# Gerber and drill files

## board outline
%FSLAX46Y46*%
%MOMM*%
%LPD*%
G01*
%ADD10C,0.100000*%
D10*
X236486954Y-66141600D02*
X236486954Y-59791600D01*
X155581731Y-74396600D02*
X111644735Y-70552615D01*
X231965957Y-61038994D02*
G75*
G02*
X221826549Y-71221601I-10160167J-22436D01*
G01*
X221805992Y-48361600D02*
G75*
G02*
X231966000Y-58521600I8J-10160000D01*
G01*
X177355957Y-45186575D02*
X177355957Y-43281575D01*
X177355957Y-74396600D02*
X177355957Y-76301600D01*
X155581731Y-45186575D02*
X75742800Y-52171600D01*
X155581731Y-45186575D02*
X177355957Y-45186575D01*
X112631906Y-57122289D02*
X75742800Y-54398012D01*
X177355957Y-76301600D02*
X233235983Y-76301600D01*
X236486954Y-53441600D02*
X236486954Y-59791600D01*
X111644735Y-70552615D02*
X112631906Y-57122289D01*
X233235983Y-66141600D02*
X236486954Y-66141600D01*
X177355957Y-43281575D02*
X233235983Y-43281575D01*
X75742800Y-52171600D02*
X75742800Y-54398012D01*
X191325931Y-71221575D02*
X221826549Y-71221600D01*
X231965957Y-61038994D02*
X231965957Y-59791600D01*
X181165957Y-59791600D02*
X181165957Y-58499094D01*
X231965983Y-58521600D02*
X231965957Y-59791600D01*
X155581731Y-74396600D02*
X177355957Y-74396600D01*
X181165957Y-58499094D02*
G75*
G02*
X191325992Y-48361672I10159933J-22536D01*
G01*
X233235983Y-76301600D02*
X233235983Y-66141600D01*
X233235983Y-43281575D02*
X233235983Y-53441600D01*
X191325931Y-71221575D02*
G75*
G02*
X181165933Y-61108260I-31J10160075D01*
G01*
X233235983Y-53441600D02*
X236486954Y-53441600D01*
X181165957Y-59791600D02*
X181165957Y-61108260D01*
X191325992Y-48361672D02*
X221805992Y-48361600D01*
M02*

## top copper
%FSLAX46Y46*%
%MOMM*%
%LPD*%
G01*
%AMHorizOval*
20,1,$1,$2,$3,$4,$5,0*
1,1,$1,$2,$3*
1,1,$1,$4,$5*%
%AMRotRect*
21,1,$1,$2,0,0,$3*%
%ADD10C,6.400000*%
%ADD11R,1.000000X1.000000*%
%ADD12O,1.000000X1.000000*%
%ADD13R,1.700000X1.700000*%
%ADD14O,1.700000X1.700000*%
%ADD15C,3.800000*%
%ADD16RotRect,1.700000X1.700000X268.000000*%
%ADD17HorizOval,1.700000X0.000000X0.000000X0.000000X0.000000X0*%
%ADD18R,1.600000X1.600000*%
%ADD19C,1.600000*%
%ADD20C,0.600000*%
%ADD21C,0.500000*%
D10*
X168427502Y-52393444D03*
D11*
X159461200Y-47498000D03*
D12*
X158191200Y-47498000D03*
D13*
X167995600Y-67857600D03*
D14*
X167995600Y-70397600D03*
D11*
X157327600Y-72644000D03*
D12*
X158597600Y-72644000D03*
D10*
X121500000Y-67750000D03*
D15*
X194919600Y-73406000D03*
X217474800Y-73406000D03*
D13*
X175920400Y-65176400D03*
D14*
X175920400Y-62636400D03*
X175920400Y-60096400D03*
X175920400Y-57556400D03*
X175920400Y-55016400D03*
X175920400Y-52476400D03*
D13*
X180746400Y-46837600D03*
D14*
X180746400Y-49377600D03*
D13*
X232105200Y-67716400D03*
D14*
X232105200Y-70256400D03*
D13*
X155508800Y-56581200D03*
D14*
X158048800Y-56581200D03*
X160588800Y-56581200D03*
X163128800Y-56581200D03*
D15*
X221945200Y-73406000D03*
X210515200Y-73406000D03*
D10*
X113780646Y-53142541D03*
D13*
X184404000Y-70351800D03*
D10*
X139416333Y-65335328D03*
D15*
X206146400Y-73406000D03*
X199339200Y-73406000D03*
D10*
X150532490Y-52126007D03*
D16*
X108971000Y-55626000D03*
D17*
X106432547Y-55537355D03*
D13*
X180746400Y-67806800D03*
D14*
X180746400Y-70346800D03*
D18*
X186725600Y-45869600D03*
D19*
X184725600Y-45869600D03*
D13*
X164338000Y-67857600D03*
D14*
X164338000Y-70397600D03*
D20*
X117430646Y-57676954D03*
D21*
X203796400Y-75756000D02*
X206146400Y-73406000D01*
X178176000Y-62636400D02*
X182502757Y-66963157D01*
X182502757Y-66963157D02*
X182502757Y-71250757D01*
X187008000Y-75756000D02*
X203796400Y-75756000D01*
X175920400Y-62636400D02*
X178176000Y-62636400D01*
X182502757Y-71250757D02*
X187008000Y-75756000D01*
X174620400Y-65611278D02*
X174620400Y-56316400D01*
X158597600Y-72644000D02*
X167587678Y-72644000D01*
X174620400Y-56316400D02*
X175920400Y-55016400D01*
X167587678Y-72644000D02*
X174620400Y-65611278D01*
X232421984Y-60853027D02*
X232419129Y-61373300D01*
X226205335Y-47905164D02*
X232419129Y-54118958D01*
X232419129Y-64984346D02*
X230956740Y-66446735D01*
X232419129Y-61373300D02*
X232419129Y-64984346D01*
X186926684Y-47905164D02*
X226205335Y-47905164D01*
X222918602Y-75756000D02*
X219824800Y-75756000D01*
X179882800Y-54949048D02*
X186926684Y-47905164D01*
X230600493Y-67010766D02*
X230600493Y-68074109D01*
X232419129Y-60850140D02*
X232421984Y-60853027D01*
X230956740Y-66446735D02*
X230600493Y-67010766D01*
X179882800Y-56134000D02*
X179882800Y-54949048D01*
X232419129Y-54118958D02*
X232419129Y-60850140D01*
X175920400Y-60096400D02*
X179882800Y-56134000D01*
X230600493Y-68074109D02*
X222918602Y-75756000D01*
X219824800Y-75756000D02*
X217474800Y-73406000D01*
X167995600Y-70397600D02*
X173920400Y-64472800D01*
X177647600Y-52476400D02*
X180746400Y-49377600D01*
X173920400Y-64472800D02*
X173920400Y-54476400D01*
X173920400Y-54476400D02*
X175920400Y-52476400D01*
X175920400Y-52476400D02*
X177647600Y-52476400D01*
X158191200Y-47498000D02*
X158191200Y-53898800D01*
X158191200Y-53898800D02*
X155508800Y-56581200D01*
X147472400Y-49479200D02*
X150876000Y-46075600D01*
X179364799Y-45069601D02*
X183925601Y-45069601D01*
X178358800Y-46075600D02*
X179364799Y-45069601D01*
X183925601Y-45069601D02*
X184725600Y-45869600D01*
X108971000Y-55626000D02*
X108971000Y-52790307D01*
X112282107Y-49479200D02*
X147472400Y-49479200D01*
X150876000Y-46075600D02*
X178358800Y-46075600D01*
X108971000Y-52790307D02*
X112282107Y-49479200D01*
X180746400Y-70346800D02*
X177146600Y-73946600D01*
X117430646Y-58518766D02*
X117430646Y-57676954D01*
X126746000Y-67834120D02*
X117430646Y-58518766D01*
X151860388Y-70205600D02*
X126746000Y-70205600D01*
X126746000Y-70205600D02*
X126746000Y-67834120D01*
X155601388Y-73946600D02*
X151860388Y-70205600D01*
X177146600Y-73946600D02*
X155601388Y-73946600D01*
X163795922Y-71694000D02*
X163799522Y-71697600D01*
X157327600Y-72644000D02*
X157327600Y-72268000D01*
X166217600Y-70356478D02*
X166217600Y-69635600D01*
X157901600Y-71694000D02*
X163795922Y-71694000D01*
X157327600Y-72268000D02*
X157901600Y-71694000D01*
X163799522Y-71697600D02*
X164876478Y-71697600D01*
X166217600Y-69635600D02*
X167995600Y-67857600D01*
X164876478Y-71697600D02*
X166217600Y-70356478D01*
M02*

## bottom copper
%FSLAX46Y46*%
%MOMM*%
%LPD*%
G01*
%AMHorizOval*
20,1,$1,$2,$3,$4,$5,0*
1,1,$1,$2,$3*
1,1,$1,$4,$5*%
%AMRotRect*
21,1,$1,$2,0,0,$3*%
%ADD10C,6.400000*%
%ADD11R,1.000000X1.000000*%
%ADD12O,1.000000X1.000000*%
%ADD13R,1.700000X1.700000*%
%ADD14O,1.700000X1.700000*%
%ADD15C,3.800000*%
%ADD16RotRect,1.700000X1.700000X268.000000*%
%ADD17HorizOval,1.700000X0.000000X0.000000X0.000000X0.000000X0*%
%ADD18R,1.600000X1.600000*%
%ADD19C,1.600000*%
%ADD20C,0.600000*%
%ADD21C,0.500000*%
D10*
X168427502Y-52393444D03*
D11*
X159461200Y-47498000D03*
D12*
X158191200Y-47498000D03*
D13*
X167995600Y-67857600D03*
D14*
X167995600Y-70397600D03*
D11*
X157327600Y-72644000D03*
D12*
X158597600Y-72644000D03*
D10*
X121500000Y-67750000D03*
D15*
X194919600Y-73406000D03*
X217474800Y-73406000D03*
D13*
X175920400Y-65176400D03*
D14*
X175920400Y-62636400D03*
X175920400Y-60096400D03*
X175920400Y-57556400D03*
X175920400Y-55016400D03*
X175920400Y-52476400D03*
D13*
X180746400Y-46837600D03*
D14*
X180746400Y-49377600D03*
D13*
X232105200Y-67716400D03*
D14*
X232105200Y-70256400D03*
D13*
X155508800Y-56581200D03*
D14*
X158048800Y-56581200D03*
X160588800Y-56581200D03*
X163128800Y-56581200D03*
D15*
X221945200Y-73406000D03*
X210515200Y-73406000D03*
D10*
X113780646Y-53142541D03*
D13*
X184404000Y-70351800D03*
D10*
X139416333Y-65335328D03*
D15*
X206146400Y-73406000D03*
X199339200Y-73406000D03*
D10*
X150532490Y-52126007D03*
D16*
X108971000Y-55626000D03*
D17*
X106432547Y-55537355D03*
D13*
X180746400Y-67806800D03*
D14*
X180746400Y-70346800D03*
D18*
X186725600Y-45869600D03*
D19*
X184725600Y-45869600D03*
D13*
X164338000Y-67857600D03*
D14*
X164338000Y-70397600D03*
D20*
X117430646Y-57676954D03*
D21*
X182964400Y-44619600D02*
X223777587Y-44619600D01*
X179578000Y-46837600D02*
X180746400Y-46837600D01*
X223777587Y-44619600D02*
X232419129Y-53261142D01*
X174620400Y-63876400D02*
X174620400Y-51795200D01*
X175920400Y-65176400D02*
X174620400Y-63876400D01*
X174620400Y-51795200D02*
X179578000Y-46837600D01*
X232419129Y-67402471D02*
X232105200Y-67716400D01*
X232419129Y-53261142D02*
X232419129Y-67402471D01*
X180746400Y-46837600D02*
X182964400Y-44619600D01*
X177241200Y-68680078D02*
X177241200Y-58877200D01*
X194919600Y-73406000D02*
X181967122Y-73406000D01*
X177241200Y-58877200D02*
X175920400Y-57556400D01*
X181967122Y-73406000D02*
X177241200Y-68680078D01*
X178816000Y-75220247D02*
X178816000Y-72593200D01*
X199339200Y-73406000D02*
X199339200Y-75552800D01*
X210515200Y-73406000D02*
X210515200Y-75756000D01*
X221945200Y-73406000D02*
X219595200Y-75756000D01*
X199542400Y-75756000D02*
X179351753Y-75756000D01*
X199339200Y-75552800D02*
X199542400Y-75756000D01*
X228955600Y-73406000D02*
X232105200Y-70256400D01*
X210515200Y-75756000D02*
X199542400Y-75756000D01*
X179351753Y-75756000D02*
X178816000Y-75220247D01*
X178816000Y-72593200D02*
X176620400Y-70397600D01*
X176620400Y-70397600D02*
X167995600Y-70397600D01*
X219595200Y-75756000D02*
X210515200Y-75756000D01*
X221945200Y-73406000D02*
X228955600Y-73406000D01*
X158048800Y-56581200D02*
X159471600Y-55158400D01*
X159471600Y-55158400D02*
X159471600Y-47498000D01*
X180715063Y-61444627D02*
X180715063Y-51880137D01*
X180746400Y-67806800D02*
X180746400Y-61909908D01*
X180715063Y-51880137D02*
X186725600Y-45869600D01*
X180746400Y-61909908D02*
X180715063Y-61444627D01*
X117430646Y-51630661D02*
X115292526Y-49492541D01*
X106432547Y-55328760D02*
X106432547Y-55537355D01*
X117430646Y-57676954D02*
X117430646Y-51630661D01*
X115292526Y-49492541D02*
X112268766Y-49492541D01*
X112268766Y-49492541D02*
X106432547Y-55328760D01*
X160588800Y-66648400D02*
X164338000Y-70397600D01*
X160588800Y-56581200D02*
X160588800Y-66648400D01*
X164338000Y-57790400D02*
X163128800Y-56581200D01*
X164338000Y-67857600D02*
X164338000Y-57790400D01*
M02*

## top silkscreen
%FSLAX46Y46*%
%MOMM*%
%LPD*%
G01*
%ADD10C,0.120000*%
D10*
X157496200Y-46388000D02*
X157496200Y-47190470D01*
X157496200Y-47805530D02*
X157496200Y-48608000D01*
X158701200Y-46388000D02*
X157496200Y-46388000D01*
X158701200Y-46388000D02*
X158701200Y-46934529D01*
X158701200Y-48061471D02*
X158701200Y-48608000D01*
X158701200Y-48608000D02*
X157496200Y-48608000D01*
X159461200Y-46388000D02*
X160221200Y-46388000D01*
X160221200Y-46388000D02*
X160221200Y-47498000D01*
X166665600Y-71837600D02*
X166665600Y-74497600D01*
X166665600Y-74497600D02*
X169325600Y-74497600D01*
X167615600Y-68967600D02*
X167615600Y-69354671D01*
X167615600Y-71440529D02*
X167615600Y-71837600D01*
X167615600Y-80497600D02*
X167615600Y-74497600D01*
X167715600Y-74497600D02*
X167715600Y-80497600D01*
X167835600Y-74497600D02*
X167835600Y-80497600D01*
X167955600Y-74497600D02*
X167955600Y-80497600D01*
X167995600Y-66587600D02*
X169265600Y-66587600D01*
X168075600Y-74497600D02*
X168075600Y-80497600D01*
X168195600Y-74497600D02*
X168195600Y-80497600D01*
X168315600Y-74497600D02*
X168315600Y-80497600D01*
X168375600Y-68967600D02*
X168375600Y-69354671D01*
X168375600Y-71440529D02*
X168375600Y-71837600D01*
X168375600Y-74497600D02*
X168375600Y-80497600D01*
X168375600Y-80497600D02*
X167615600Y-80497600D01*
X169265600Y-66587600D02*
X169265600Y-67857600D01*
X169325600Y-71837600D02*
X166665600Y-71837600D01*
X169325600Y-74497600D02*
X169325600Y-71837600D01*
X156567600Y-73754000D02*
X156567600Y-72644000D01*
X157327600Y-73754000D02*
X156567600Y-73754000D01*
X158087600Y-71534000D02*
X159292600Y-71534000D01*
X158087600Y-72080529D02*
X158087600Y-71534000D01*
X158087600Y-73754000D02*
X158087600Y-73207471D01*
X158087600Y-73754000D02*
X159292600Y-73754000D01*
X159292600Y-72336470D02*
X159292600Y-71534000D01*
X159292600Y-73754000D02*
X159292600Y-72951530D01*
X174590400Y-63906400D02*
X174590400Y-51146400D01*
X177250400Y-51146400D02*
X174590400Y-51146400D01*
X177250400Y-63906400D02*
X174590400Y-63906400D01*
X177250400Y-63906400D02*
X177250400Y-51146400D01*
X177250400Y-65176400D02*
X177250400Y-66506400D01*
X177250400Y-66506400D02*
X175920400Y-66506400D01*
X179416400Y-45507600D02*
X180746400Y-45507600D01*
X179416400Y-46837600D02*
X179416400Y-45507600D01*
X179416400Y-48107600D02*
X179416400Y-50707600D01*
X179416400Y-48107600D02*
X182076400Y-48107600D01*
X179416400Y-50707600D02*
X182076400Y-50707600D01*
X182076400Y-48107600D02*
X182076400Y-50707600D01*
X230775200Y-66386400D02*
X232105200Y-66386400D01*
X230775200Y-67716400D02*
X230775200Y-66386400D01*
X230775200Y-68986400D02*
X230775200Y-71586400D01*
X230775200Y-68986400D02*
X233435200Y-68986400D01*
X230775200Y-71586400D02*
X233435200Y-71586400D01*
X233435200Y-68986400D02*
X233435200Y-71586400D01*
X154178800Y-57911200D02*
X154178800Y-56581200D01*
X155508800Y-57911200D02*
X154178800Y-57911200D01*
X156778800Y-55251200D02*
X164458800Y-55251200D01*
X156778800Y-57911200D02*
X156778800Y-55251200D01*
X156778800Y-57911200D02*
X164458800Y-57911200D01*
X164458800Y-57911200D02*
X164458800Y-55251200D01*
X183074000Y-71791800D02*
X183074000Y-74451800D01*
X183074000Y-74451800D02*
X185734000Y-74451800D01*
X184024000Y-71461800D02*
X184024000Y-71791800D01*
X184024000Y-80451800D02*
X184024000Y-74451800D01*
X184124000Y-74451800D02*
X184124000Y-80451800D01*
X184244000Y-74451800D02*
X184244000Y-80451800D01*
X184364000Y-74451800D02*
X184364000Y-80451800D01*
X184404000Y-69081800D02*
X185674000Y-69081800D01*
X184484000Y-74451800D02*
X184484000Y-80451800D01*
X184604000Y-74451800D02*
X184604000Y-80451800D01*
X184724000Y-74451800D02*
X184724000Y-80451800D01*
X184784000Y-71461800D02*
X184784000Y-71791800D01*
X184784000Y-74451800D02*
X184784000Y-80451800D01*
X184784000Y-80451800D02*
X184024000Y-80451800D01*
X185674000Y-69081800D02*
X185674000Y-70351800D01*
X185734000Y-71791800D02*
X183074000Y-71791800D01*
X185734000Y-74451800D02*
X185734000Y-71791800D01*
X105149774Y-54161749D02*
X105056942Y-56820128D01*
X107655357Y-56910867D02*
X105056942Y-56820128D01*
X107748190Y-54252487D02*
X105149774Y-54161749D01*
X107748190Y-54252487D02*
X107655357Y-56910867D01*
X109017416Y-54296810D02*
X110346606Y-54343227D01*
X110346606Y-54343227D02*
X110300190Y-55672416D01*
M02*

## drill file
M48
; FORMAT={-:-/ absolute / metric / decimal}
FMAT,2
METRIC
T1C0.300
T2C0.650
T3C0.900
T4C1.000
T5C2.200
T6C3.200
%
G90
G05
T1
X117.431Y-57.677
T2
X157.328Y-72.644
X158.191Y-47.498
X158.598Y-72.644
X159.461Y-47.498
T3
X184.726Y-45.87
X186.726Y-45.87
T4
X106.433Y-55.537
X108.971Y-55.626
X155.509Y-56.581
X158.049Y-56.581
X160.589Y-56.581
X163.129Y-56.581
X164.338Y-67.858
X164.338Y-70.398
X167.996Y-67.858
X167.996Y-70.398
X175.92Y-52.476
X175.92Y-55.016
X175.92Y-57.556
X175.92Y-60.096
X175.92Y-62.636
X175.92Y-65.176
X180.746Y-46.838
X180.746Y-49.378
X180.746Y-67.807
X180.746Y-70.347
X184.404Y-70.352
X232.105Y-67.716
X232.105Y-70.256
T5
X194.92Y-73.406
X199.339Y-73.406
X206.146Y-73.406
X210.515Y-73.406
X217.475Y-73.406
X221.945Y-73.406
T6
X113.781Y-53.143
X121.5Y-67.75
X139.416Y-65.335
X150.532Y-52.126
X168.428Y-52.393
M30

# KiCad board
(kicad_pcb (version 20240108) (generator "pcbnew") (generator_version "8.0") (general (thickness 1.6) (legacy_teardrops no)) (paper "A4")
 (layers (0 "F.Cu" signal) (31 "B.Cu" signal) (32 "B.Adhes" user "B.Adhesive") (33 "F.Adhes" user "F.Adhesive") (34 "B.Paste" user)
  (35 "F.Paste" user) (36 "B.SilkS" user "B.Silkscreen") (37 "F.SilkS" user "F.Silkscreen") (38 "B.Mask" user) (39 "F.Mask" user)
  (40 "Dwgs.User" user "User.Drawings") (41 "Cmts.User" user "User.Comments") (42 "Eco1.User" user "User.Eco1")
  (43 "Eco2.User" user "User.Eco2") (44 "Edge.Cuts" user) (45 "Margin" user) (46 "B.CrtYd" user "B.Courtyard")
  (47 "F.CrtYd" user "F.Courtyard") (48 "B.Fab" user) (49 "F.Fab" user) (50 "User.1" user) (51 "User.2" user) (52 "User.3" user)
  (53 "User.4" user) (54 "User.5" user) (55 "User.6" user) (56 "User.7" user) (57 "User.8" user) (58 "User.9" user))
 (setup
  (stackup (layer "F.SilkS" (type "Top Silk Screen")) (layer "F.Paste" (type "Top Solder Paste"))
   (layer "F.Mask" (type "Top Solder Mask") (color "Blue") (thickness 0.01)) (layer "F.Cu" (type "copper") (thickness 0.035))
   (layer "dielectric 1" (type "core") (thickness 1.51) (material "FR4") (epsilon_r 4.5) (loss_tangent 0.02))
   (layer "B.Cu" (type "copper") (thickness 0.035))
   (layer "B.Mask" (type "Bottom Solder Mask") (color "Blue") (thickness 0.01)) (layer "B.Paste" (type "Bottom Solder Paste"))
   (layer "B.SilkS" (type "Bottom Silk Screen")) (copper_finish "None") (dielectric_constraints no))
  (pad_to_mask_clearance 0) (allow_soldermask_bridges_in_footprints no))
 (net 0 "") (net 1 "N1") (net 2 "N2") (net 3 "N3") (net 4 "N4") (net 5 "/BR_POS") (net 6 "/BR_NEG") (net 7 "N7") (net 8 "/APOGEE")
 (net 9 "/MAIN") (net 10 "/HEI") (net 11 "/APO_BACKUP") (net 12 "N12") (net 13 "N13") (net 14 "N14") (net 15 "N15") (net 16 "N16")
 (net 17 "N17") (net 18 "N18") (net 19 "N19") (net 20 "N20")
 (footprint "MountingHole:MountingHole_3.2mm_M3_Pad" (layer "F.Cu") (at 168.427502 52.393444)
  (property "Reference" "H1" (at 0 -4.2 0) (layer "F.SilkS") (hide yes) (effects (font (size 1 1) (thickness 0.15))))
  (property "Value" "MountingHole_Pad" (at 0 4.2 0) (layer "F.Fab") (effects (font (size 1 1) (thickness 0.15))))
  (pad "1" thru_hole circle (at 0 0) (size 6.4 6.4) (drill 3.2) (layers "*.Cu" "*.Mask") (remove_unused_layers no) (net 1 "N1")))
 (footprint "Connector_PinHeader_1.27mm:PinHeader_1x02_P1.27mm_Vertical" (layer "F.Cu") (at 159.4612 47.498 -90)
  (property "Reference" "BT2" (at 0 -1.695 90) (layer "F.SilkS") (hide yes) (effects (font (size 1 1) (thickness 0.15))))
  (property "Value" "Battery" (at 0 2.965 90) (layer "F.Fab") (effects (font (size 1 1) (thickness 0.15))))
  (fp_line (start -1.11 1.965) (end -0.30753 1.965) (stroke (width 0.12) (type solid)) (layer "F.SilkS"))
  (fp_line (start 0.30753 1.965) (end 1.11 1.965) (stroke (width 0.12) (type solid)) (layer "F.SilkS"))
  (fp_line (start -1.11 0.76) (end -1.11 1.965) (stroke (width 0.12) (type solid)) (layer "F.SilkS"))
  (fp_line (start -1.11 0.76) (end -0.563471 0.76) (stroke (width 0.12) (type solid)) (layer "F.SilkS"))
  (fp_line (start 0.563471 0.76) (end 1.11 0.76) (stroke (width 0.12) (type solid)) (layer "F.SilkS"))
  (fp_line (start 1.11 0.76) (end 1.11 1.965) (stroke (width 0.12) (type solid)) (layer "F.SilkS"))
  (fp_line (start -1.11 0) (end -1.11 -0.76) (stroke (width 0.12) (type solid)) (layer "F.SilkS"))
  (fp_line (start -1.11 -0.76) (end 0 -0.76) (stroke (width 0.12) (type solid)) (layer "F.SilkS"))
  (pad "1" thru_hole rect (at 0 0 270) (size 1 1) (drill 0.65) (layers "*.Cu" "*.Mask") (remove_unused_layers no) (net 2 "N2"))
  (pad "2" thru_hole oval (at 0 1.27 270) (size 1 1) (drill 0.65) (layers "*.Cu" "*.Mask") (remove_unused_layers no) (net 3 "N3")))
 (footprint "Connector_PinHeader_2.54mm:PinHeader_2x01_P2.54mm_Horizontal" (layer "F.Cu") (at 167.9956 67.8576 -90)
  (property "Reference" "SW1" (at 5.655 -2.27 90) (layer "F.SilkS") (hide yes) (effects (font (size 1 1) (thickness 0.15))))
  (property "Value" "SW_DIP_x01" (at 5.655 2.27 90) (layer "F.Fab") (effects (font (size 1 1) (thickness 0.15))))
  (fp_line (start 3.98 1.33) (end 6.64 1.33) (stroke (width 0.12) (type solid)) (layer "F.SilkS"))
  (fp_line (start 6.64 1.33) (end 6.64 -1.33) (stroke (width 0.12) (type solid)) (layer "F.SilkS"))
  (fp_line (start 1.11 0.38) (end 1.497071 0.38) (stroke (width 0.12) (type solid)) (layer "F.SilkS"))
  (fp_line (start 3.582929 0.38) (end 3.98 0.38) (stroke (width 0.12) (type solid)) (layer "F.SilkS"))
  (fp_line (start 12.64 0.38) (end 6.64 0.38) (stroke (width 0.12) (type solid)) (layer "F.SilkS"))
  (fp_line (start 6.64 0.28) (end 12.64 0.28) (stroke (width 0.12) (type solid)) (layer "F.SilkS"))
  (fp_line (start 6.64 0.16) (end 12.64 0.16) (stroke (width 0.12) (type solid)) (layer "F.SilkS"))
  (fp_line (start 6.64 0.04) (end 12.64 0.04) (stroke (width 0.12) (type solid)) (layer "F.SilkS"))
  (fp_line (start -1.27 0) (end -1.27 -1.27) (stroke (width 0.12) (type solid)) (layer "F.SilkS"))
  (fp_line (start 6.64 -0.08) (end 12.64 -0.08) (stroke (width 0.12) (type solid)) (layer "F.SilkS"))
  (fp_line (start 6.64 -0.2) (end 12.64 -0.2) (stroke (width 0.12) (type solid)) (layer "F.SilkS"))
  (fp_line (start 6.64 -0.32) (end 12.64 -0.32) (stroke (width 0.12) (type solid)) (layer "F.SilkS"))
  (fp_line (start 1.11 -0.38) (end 1.497071 -0.38) (stroke (width 0.12) (type solid)) (layer "F.SilkS"))
  (fp_line (start 3.582929 -0.38) (end 3.98 -0.38) (stroke (width 0.12) (type solid)) (layer "F.SilkS"))
  (fp_line (start 6.64 -0.38) (end 12.64 -0.38) (stroke (width 0.12) (type solid)) (layer "F.SilkS"))
  (fp_line (start 12.64 -0.38) (end 12.64 0.38) (stroke (width 0.12) (type solid)) (layer "F.SilkS"))
  (fp_line (start -1.27 -1.27) (end 0 -1.27) (stroke (width 0.12) (type solid)) (layer "F.SilkS"))
  (fp_line (start 3.98 -1.33) (end 3.98 1.33) (stroke (width 0.12) (type solid)) (layer "F.SilkS"))
  (fp_line (start 6.64 -1.33) (end 3.98 -1.33) (stroke (width 0.12) (type solid)) (layer "F.SilkS"))
  (pad "1" thru_hole rect (at 0 0 270) (size 1.7 1.7) (drill 1) (layers "*.Cu" "*.Mask") (remove_unused_layers no) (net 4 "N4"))
  (pad "2" thru_hole oval (at 2.54 0 270) (size 1.7 1.7) (drill 1) (layers "*.Cu" "*.Mask") (remove_unused_layers no) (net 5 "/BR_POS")))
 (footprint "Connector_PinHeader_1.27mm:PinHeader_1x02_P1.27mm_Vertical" (layer "F.Cu") (at 157.3276 72.644 90)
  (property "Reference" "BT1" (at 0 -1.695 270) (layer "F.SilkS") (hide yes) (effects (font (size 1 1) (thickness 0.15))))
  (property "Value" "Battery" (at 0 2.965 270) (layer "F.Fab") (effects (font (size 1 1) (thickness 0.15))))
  (fp_line (start -1.11 -0.76) (end 0 -0.76) (stroke (width 0.12) (type solid)) (layer "F.SilkS"))
  (fp_line (start -1.11 0) (end -1.11 -0.76) (stroke (width 0.12) (type solid)) (layer "F.SilkS"))
  (fp_line (start 1.11 0.76) (end 1.11 1.965) (stroke (width 0.12) (type solid)) (layer "F.SilkS"))
  (fp_line (start 0.563471 0.76) (end 1.11 0.76) (stroke (width 0.12) (type solid)) (layer "F.SilkS"))
  (fp_line (start -1.11 0.76) (end -0.563471 0.76) (stroke (width 0.12) (type solid)) (layer "F.SilkS"))
  (fp_line (start -1.11 0.76) (end -1.11 1.965) (stroke (width 0.12) (type solid)) (layer "F.SilkS"))
  (fp_line (start 0.30753 1.965) (end 1.11 1.965) (stroke (width 0.12) (type solid)) (layer "F.SilkS"))
  (fp_line (start -1.11 1.965) (end -0.30753 1.965) (stroke (width 0.12) (type solid)) (layer "F.SilkS"))
  (pad "1" thru_hole rect (at 0 0 90) (size 1 1) (drill 0.65) (layers "*.Cu" "*.Mask") (remove_unused_layers no) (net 4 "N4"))
  (pad "2" thru_hole oval (at 0 1.27 90) (size 1 1) (drill 0.65) (layers "*.Cu" "*.Mask") (remove_unused_layers no) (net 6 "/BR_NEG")))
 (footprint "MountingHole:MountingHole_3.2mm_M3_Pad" (layer "F.Cu") (at 121.5 67.75)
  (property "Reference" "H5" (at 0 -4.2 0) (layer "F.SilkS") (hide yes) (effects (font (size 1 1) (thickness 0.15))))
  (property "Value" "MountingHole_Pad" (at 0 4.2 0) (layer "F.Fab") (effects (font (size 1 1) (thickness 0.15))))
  (pad "1" thru_hole circle (at 0 0) (size 6.4 6.4) (drill 3.2) (layers "*.Cu" "*.Mask") (remove_unused_layers no) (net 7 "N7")))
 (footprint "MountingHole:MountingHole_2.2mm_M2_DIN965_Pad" (layer "F.Cu") (at 194.9196 73.406)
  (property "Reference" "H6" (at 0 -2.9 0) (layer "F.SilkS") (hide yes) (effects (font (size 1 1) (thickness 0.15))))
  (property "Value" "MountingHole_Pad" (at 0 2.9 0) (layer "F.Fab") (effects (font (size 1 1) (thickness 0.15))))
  (pad "1" thru_hole circle (at 0 0) (size 3.8 3.8) (drill 2.2) (layers "*.Cu" "*.Mask") (remove_unused_layers no) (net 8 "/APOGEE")))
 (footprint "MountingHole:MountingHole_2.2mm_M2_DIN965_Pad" (layer "F.Cu") (at 217.4748 73.406)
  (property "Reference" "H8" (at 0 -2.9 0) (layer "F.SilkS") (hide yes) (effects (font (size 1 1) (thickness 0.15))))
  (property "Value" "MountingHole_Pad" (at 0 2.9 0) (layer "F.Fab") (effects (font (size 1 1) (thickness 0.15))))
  (pad "1" thru_hole circle (at 0 0) (size 3.8 3.8) (drill 2.2) (layers "*.Cu" "*.Mask") (remove_unused_layers no) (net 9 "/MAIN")))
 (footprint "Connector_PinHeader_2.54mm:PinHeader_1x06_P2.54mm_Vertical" (layer "F.Cu") (at 175.9204 65.1764 180)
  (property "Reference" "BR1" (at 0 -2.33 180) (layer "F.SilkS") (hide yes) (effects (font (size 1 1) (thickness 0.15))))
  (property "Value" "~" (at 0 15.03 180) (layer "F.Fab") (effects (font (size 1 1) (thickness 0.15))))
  (fp_line (start 1.33 1.27) (end 1.33 14.03) (stroke (width 0.12) (type solid)) (layer "F.SilkS"))
  (fp_line (start -1.33 14.03) (end 1.33 14.03) (stroke (width 0.12) (type solid)) (layer "F.SilkS"))
  (fp_line (start -1.33 1.27) (end 1.33 1.27) (stroke (width 0.12) (type solid)) (layer "F.SilkS"))
  (fp_line (start -1.33 1.27) (end -1.33 14.03) (stroke (width 0.12) (type solid)) (layer "F.SilkS"))
  (fp_line (start -1.33 0) (end -1.33 -1.33) (stroke (width 0.12) (type solid)) (layer "F.SilkS"))
  (fp_line (start -1.33 -1.33) (end 0 -1.33) (stroke (width 0.12) (type solid)) (layer "F.SilkS"))
  (pad "1" thru_hole rect (at 0 0 180) (size 1.7 1.7) (drill 1) (layers "*.Cu" "*.Mask") (remove_unused_layers no) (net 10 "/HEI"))
  (pad "2" thru_hole oval (at 0 2.54 180) (size 1.7 1.7) (drill 1) (layers "*.Cu" "*.Mask") (remove_unused_layers no) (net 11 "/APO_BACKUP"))
  (pad "3" thru_hole oval (at 0 5.08 180) (size 1.7 1.7) (drill 1) (layers "*.Cu" "*.Mask") (remove_unused_layers no) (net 9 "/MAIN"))
  (pad "4" thru_hole oval (at 0 7.62 180) (size 1.7 1.7) (drill 1) (layers "*.Cu" "*.Mask") (remove_unused_layers no) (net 8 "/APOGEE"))
  (pad "5" thru_hole oval (at 0 10.16 180) (size 1.7 1.7) (drill 1) (layers "*.Cu" "*.Mask") (remove_unused_layers no) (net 6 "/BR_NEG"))
  (pad "6" thru_hole oval (at 0 12.7 180) (size 1.7 1.7) (drill 1) (layers "*.Cu" "*.Mask") (remove_unused_layers no) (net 5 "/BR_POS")))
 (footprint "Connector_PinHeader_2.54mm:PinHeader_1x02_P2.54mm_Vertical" (layer "F.Cu") (at 180.7464 46.8376)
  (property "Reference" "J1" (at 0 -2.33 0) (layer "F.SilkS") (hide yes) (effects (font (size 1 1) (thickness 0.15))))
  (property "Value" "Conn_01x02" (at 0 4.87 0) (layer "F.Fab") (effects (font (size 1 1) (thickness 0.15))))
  (fp_line (start -1.33 -1.33) (end 0 -1.33) (stroke (width 0.12) (type solid)) (layer "F.SilkS"))
  (fp_line (start -1.33 0) (end -1.33 -1.33) (stroke (width 0.12) (type solid)) (layer "F.SilkS"))
  (fp_line (start -1.33 1.27) (end -1.33 3.87) (stroke (width 0.12) (type solid)) (layer "F.SilkS"))
  (fp_line (start -1.33 1.27) (end 1.33 1.27) (stroke (width 0.12) (type solid)) (layer "F.SilkS"))
  (fp_line (start -1.33 3.87) (end 1.33 3.87) (stroke (width 0.12) (type solid)) (layer "F.SilkS"))
  (fp_line (start 1.33 1.27) (end 1.33 3.87) (stroke (width 0.12) (type solid)) (layer "F.SilkS"))
  (pad "1" thru_hole rect (at 0 0) (size 1.7 1.7) (drill 1) (layers "*.Cu" "*.Mask") (remove_unused_layers no) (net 10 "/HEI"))
  (pad "2" thru_hole oval (at 0 2.54) (size 1.7 1.7) (drill 1) (layers "*.Cu" "*.Mask") (remove_unused_layers no) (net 5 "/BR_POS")))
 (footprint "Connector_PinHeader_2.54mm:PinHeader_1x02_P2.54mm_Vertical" (layer "F.Cu") (at 232.1052 67.7164)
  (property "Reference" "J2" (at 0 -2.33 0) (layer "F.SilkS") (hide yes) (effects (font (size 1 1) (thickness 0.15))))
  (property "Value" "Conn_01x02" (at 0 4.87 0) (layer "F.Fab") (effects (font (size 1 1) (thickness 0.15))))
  (fp_line (start -1.33 -1.33) (end 0 -1.33) (stroke (width 0.12) (type solid)) (layer "F.SilkS"))
  (fp_line (start -1.33 0) (end -1.33 -1.33) (stroke (width 0.12) (type solid)) (layer "F.SilkS"))
  (fp_line (start -1.33 1.27) (end -1.33 3.87) (stroke (width 0.12) (type solid)) (layer "F.SilkS"))
  (fp_line (start -1.33 1.27) (end 1.33 1.27) (stroke (width 0.12) (type solid)) (layer "F.SilkS"))
  (fp_line (start -1.33 3.87) (end 1.33 3.87) (stroke (width 0.12) (type solid)) (layer "F.SilkS"))
  (fp_line (start 1.33 1.27) (end 1.33 3.87) (stroke (width 0.12) (type solid)) (layer "F.SilkS"))
  (pad "1" thru_hole rect (at 0 0) (size 1.7 1.7) (drill 1) (layers "*.Cu" "*.Mask") (remove_unused_layers no) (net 10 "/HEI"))
  (pad "2" thru_hole oval (at 0 2.54) (size 1.7 1.7) (drill 1) (layers "*.Cu" "*.Mask") (remove_unused_layers no) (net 5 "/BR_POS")))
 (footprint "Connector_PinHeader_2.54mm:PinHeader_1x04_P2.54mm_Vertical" (layer "F.Cu") (at 155.5088 56.5812 90)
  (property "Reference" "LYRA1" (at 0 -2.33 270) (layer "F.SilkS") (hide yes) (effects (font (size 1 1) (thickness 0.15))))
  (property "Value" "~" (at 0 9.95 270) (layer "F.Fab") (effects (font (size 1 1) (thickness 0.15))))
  (fp_line (start -1.33 -1.33) (end 0 -1.33) (stroke (width 0.12) (type solid)) (layer "F.SilkS"))
  (fp_line (start -1.33 0) (end -1.33 -1.33) (stroke (width 0.12) (type solid)) (layer "F.SilkS"))
  (fp_line (start 1.33 1.27) (end 1.33 8.95) (stroke (width 0.12) (type solid)) (layer "F.SilkS"))
  (fp_line (start -1.33 1.27) (end 1.33 1.27) (stroke (width 0.12) (type solid)) (layer "F.SilkS"))
  (fp_line (start -1.33 1.27) (end -1.33 8.95) (stroke (width 0.12) (type solid)) (layer "F.SilkS"))
  (fp_line (start -1.33 8.95) (end 1.33 8.95) (stroke (width 0.12) (type solid)) (layer "F.SilkS"))
  (pad "1" thru_hole rect (at 0 0 90) (size 1.7 1.7) (drill 1) (layers "*.Cu" "*.Mask") (remove_unused_layers no) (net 3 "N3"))
  (pad "2" thru_hole oval (at 0 2.54 90) (size 1.7 1.7) (drill 1) (layers "*.Cu" "*.Mask") (remove_unused_layers no) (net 2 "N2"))
  (pad "3" thru_hole oval (at 0 5.08 90) (size 1.7 1.7) (drill 1) (layers "*.Cu" "*.Mask") (remove_unused_layers no) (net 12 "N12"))
  (pad "4" thru_hole oval (at 0 7.62 90) (size 1.7 1.7) (drill 1) (layers "*.Cu" "*.Mask") (remove_unused_layers no) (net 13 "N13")))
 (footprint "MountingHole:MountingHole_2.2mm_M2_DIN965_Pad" (layer "F.Cu") (at 221.9452 73.406)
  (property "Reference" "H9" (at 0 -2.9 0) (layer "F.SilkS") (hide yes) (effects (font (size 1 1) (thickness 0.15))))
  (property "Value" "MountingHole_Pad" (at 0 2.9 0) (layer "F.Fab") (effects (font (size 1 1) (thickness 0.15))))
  (pad "1" thru_hole circle (at 0 0) (size 3.8 3.8) (drill 2.2) (layers "*.Cu" "*.Mask") (remove_unused_layers no) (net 5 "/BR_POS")))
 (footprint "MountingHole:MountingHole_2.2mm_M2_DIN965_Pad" (layer "F.Cu") (at 210.5152 73.406)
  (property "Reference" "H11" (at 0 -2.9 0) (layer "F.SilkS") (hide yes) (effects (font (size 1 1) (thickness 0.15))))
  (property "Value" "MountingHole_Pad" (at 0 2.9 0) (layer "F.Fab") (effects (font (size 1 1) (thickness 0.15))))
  (pad "1" thru_hole circle (at 0 0) (size 3.8 3.8) (drill 2.2) (layers "*.Cu" "*.Mask") (remove_unused_layers no) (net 5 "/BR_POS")))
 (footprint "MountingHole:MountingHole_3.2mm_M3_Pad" (layer "F.Cu") (at 113.780646 53.142541)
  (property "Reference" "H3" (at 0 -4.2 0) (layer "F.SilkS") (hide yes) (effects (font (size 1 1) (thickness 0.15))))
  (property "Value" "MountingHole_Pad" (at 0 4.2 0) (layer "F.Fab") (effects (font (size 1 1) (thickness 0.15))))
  (pad "1" thru_hole circle (at 0 0) (size 6.4 6.4) (drill 3.2) (layers "*.Cu" "*.Mask") (remove_unused_layers no) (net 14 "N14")))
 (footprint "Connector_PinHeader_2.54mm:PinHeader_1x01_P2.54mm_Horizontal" (layer "F.Cu") (at 184.404 70.3518 -90)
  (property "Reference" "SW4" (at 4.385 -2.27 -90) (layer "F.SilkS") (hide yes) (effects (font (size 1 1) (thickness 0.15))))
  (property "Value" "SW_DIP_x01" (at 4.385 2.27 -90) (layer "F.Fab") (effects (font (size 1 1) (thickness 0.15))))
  (fp_line (start 1.44 1.33) (end 4.1 1.33) (stroke (width 0.12) (type solid)) (layer "F.SilkS"))
  (fp_line (start 4.1 1.33) (end 4.1 -1.33) (stroke (width 0.12) (type solid)) (layer "F.SilkS"))
  (fp_line (start 1.11 0.38) (end 1.44 0.38) (stroke (width 0.12) (type solid)) (layer "F.SilkS"))
  (fp_line (start 10.1 0.38) (end 4.1 0.38) (stroke (width 0.12) (type solid)) (layer "F.SilkS"))
  (fp_line (start 4.1 0.28) (end 10.1 0.28) (stroke (width 0.12) (type solid)) (layer "F.SilkS"))
  (fp_line (start 4.1 0.16) (end 10.1 0.16) (stroke (width 0.12) (type solid)) (layer "F.SilkS"))
  (fp_line (start 4.1 0.04) (end 10.1 0.04) (stroke (width 0.12) (type solid)) (layer "F.SilkS"))
  (fp_line (start -1.27 0) (end -1.27 -1.27) (stroke (width 0.12) (type solid)) (layer "F.SilkS"))
  (fp_line (start 4.1 -0.08) (end 10.1 -0.08) (stroke (width 0.12) (type solid)) (layer "F.SilkS"))
  (fp_line (start 4.1 -0.2) (end 10.1 -0.2) (stroke (width 0.12) (type solid)) (layer "F.SilkS"))
  (fp_line (start 4.1 -0.32) (end 10.1 -0.32) (stroke (width 0.12) (type solid)) (layer "F.SilkS"))
  (fp_line (start 1.11 -0.38) (end 1.44 -0.38) (stroke (width 0.12) (type solid)) (layer "F.SilkS"))
  (fp_line (start 4.1 -0.38) (end 10.1 -0.38) (stroke (width 0.12) (type solid)) (layer "F.SilkS"))
  (fp_line (start 10.1 -0.38) (end 10.1 0.38) (stroke (width 0.12) (type solid)) (layer "F.SilkS"))
  (fp_line (start -1.27 -1.27) (end 0 -1.27) (stroke (width 0.12) (type solid)) (layer "F.SilkS"))
  (fp_line (start 1.44 -1.33) (end 1.44 1.33) (stroke (width 0.12) (type solid)) (layer "F.SilkS"))
  (fp_line (start 4.1 -1.33) (end 1.44 -1.33) (stroke (width 0.12) (type solid)) (layer "F.SilkS"))
  (pad "1" thru_hole rect (at 0 0 270) (size 1.7 1.7) (drill 1) (layers "*.Cu" "*.Mask") (remove_unused_layers no) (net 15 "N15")))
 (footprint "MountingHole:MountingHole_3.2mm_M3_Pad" (layer "F.Cu") (at 139.416333 65.335328)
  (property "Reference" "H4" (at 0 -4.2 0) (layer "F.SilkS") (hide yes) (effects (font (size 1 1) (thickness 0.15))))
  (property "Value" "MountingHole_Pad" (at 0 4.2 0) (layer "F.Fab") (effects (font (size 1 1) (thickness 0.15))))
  (pad "1" thru_hole circle (at 0 0) (size 6.4 6.4) (drill 3.2) (layers "*.Cu" "*.Mask") (remove_unused_layers no) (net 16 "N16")))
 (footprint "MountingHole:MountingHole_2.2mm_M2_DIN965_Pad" (layer "F.Cu") (at 206.1464 73.406)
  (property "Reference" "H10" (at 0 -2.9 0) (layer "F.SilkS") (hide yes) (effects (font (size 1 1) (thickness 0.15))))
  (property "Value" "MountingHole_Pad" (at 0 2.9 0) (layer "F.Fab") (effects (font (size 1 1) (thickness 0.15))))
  (pad "1" thru_hole circle (at 0 0) (size 3.8 3.8) (drill 2.2) (layers "*.Cu" "*.Mask") (remove_unused_layers no) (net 11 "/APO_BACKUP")))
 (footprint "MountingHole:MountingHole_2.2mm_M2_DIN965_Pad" (layer "F.Cu") (at 199.3392 73.406)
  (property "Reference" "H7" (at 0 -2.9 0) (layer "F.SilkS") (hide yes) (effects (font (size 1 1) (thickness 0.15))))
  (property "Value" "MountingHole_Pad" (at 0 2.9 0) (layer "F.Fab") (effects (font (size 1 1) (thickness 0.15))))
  (pad "1" thru_hole circle (at 0 0) (size 3.8 3.8) (drill 2.2) (layers "*.Cu" "*.Mask") (remove_unused_layers no) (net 5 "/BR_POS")))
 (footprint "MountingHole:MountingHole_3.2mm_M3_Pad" (layer "F.Cu") (at 150.53249 52.126007)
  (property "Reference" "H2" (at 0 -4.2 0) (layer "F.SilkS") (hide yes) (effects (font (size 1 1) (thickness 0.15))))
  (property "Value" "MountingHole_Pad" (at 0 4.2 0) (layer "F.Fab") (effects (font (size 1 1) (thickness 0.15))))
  (pad "1" thru_hole circle (at 0 0) (size 6.4 6.4) (drill 3.2) (layers "*.Cu" "*.Mask") (remove_unused_layers no) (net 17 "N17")))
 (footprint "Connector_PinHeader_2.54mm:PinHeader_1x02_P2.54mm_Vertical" (layer "F.Cu") (at 108.971 55.626 -92)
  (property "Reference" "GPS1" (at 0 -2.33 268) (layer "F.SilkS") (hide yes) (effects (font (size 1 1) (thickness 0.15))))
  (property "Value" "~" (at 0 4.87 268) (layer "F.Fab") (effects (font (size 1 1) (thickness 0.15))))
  (fp_line (start -1.33 3.87) (end 1.329999 3.869999) (stroke (width 0.12) (type solid)) (layer "F.SilkS"))
  (fp_line (start 1.33 1.27) (end 1.329999 3.869999) (stroke (width 0.12) (type solid)) (layer "F.SilkS"))
  (fp_line (start -1.330001 1.27) (end -1.33 3.87) (stroke (width 0.12) (type solid)) (layer "F.SilkS"))
  (fp_line (start -1.330001 1.27) (end 1.33 1.27) (stroke (width 0.12) (type solid)) (layer "F.SilkS"))
  (fp_line (start -1.33 0) (end -1.33 -1.33) (stroke (width 0.12) (type solid)) (layer "F.SilkS"))
  (fp_line (start -1.33 -1.33) (end 0 -1.33) (stroke (width 0.12) (type solid)) (layer "F.SilkS"))
  (pad "1" thru_hole rect (at 0 0 268) (size 1.7 1.7) (drill 1) (layers "*.Cu" "*.Mask") (remove_unused_layers no) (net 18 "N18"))
  (pad "2" thru_hole oval (at 0 2.54 268) (size 1.7 1.7) (drill 1) (layers "*.Cu" "*.Mask") (remove_unused_layers no) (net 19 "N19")))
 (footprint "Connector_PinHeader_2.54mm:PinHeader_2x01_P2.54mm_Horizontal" (layer "B.Cu") (at 180.7464 67.8068 -90)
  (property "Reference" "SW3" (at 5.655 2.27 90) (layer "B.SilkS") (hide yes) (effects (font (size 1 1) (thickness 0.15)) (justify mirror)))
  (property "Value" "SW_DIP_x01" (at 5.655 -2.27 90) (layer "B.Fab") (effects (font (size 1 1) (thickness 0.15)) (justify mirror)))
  (pad "1" thru_hole rect (at 0 0 270) (size 1.7 1.7) (drill 1) (layers "*.Cu" "*.Mask") (remove_unused_layers no) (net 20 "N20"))
  (pad "2" thru_hole oval (at 2.54 0 270) (size 1.7 1.7) (drill 1) (layers "*.Cu" "*.Mask") (remove_unused_layers no) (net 19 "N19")))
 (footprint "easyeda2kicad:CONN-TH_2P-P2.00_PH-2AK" (layer "B.Cu") (at 185.7256 45.8696 180)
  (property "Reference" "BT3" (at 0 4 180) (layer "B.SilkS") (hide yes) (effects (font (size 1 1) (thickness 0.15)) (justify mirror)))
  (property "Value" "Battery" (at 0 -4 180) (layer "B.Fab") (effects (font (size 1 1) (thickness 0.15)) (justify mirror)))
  (pad "1" thru_hole rect (at -1 0 180) (size 1.6 1.6) (drill 0.900024) (layers "*.Cu" "*.Mask") (remove_unused_layers no) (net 20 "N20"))
  (pad "2" thru_hole circle (at 1 0 180) (size 1.6 1.6) (drill 0.900024) (layers "*.Cu" "*.Mask") (remove_unused_layers no) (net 18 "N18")))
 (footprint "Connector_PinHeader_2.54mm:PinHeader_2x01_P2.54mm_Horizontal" (layer "B.Cu") (at 164.338 67.8576 -90)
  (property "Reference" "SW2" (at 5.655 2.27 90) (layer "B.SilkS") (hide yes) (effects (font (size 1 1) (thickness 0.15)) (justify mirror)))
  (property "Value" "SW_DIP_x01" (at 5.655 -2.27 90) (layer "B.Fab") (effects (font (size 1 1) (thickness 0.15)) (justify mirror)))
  (pad "1" thru_hole rect (at 0 0 270) (size 1.7 1.7) (drill 1) (layers "*.Cu" "*.Mask") (remove_unused_layers no) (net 13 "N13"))
  (pad "2" thru_hole oval (at 2.54 0 270) (size 1.7 1.7) (drill 1) (layers "*.Cu" "*.Mask") (remove_unused_layers no) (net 12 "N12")))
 (gr_line (start 236.486954 66.1416) (end 236.486954 59.7916) (stroke (width 0.1) (type default)) (layer "Edge.Cuts"))
 (gr_line (start 155.581731 74.3966) (end 111.644735 70.552615) (stroke (width 0.1) (type default)) (layer "Edge.Cuts"))
 (gr_arc (start 231.965957 61.038994) (mid 229.005387 68.230483) (end 221.826549 71.2216) (stroke (width 0.1) (type default))
  (layer "Edge.Cuts"))
 (gr_arc (start 221.805992 48.3616) (mid 228.990173 51.337399) (end 231.965983 58.5216) (stroke (width 0.1) (type default))
  (layer "Edge.Cuts"))
 (gr_line (start 177.355957 45.186575) (end 177.355957 43.281575) (stroke (width 0.1) (type default)) (layer "Edge.Cuts"))
 (gr_line (start 177.355957 74.3966) (end 177.355957 76.3016) (stroke (width 0.1) (type default)) (layer "Edge.Cuts"))
 (gr_line (start 155.581731 45.186575) (end 75.7428 52.1716) (stroke (width 0.1) (type default)) (layer "Edge.Cuts"))
 (gr_line (start 155.581731 45.186575) (end 177.355957 45.186575) (stroke (width 0.1) (type default)) (layer "Edge.Cuts"))
 (gr_line (start 112.631906 57.122289) (end 75.7428 54.398012) (stroke (width 0.1) (type default)) (layer "Edge.Cuts"))
 (gr_line (start 177.355957 76.3016) (end 233.235983 76.3016) (stroke (width 0.1) (type default)) (layer "Edge.Cuts"))
 (gr_line (start 236.486954 53.4416) (end 236.486954 59.7916) (stroke (width 0.1) (type default)) (layer "Edge.Cuts"))
 (gr_line (start 111.644735 70.552615) (end 112.631906 57.122289) (stroke (width 0.1) (type default)) (layer "Edge.Cuts"))
 (gr_line (start 233.235983 66.1416) (end 236.486954 66.1416) (stroke (width 0.1) (type default)) (layer "Edge.Cuts"))
 (gr_line (start 177.355957 43.281575) (end 233.235983 43.281575) (stroke (width 0.1) (type default)) (layer "Edge.Cuts"))
 (gr_line (start 75.7428 52.1716) (end 75.7428 54.398012) (stroke (width 0.1) (type default)) (layer "Edge.Cuts"))
 (gr_line (start 191.325931 71.221575) (end 221.826549 71.2216) (stroke (width 0.1) (type default)) (layer "Edge.Cuts"))
 (gr_line (start 231.965957 61.038994) (end 231.965957 59.7916) (stroke (width 0.1) (type default)) (layer "Edge.Cuts"))
 (gr_line (start 181.165957 59.7916) (end 181.165957 58.499094) (stroke (width 0.1) (type default)) (layer "Edge.Cuts"))
 (gr_line (start 231.965983 58.5216) (end 231.965957 59.7916) (stroke (width 0.1) (type default)) (layer "Edge.Cuts"))
 (gr_line (start 155.581731 74.3966) (end 177.355957 74.3966) (stroke (width 0.1) (type default)) (layer "Edge.Cuts"))
 (gr_arc (start 181.165957 58.499094) (mid 184.149724 51.329456) (end 191.325992 48.361672) (stroke (width 0.1) (type default))
  (layer "Edge.Cuts"))
 (gr_line (start 233.235983 76.3016) (end 233.235983 66.1416) (stroke (width 0.1) (type default)) (layer "Edge.Cuts"))
 (gr_line (start 233.235983 43.281575) (end 233.235983 53.4416) (stroke (width 0.1) (type default)) (layer "Edge.Cuts"))
 (gr_arc (start 191.325931 71.221575) (mid 184.15821 68.262283) (end 181.165957 61.10826) (stroke (width 0.1) (type default))
  (layer "Edge.Cuts"))
 (gr_line (start 233.235983 53.4416) (end 236.486954 53.4416) (stroke (width 0.1) (type default)) (layer "Edge.Cuts"))
 (gr_line (start 181.165957 59.7916) (end 181.165957 61.10826) (stroke (width 0.1) (type default)) (layer "Edge.Cuts"))
 (gr_line (start 191.325992 48.361672) (end 221.805992 48.3616) (stroke (width 0.1) (type default)) (layer "Edge.Cuts"))
 (segment (start 182.9644 44.6196) (end 223.777587 44.6196) (width 0.5) (layer "B.Cu") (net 10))
 (segment (start 179.578 46.8376) (end 180.7464 46.8376) (width 0.5) (layer "B.Cu") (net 10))
 (segment (start 223.777587 44.6196) (end 232.419129 53.261142) (width 0.5) (layer "B.Cu") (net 10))
 (segment (start 174.6204 63.8764) (end 174.6204 51.7952) (width 0.5) (layer "B.Cu") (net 10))
 (segment (start 175.9204 65.1764) (end 174.6204 63.8764) (width 0.5) (layer "B.Cu") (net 10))
 (segment (start 174.6204 51.7952) (end 179.578 46.8376) (width 0.5) (layer "B.Cu") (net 10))
 (segment (start 232.419129 67.402471) (end 232.1052 67.7164) (width 0.5) (layer "B.Cu") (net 10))
 (segment (start 232.419129 53.261142) (end 232.419129 67.402471) (width 0.5) (layer "B.Cu") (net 10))
 (segment (start 180.7464 46.8376) (end 182.9644 44.6196) (width 0.5) (layer "B.Cu") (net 10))
 (segment (start 203.7964 75.756) (end 206.1464 73.406) (width 0.5) (layer "F.Cu") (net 11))
 (segment (start 178.176 62.6364) (end 182.502757 66.963157) (width 0.5) (layer "F.Cu") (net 11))
 (segment (start 182.502757 66.963157) (end 182.502757 71.250757) (width 0.5) (layer "F.Cu") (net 11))
 (segment (start 187.008 75.756) (end 203.7964 75.756) (width 0.5) (layer "F.Cu") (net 11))
 (segment (start 175.9204 62.6364) (end 178.176 62.6364) (width 0.5) (layer "F.Cu") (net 11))
 (segment (start 182.502757 71.250757) (end 187.008 75.756) (width 0.5) (layer "F.Cu") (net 11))
 (segment (start 177.2412 68.680078) (end 177.2412 58.8772) (width 0.5) (layer "B.Cu") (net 8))
 (segment (start 194.9196 73.406) (end 181.967122 73.406) (width 0.5) (layer "B.Cu") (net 8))
 (segment (start 177.2412 58.8772) (end 175.9204 57.5564) (width 0.5) (layer "B.Cu") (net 8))
 (segment (start 181.967122 73.406) (end 177.2412 68.680078) (width 0.5) (layer "B.Cu") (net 8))
 (segment (start 174.6204 65.611278) (end 174.6204 56.3164) (width 0.5) (layer "F.Cu") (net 6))
 (segment (start 158.5976 72.644) (end 167.587678 72.644) (width 0.5) (layer "F.Cu") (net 6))
 (segment (start 174.6204 56.3164) (end 175.9204 55.0164) (width 0.5) (layer "F.Cu") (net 6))
 (segment (start 167.587678 72.644) (end 174.6204 65.611278) (width 0.5) (layer "F.Cu") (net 6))
 (segment (start 232.421984 60.853027) (end 232.419129 61.3733) (width 0.5) (layer "F.Cu") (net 9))
 (segment (start 226.205335 47.905164) (end 232.419129 54.118958) (width 0.5) (layer "F.Cu") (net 9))
 (segment (start 232.419129 64.984346) (end 230.95674 66.446735) (width 0.5) (layer "F.Cu") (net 9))
 (segment (start 232.419129 61.3733) (end 232.419129 64.984346) (width 0.5) (layer "F.Cu") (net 9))
 (segment (start 186.926684 47.905164) (end 226.205335 47.905164) (width 0.5) (layer "F.Cu") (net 9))
 (segment (start 222.918602 75.756) (end 219.8248 75.756) (width 0.5) (layer "F.Cu") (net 9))
 (segment (start 179.8828 54.949048) (end 186.926684 47.905164) (width 0.5) (layer "F.Cu") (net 9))
 (segment (start 230.600493 67.010766) (end 230.600493 68.074109) (width 0.5) (layer "F.Cu") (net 9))
 (segment (start 232.419129 60.85014) (end 232.421984 60.853027) (width 0.5) (layer "F.Cu") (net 9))
 (segment (start 230.95674 66.446735) (end 230.600493 67.010766) (width 0.5) (layer "F.Cu") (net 9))
 (segment (start 179.8828 56.134) (end 179.8828 54.949048) (width 0.5) (layer "F.Cu") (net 9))
 (segment (start 232.419129 54.118958) (end 232.419129 60.85014) (width 0.5) (layer "F.Cu") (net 9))
 (segment (start 175.9204 60.0964) (end 179.8828 56.134) (width 0.5) (layer "F.Cu") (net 9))
 (segment (start 230.600493 68.074109) (end 222.918602 75.756) (width 0.5) (layer "F.Cu") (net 9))
 (segment (start 219.8248 75.756) (end 217.4748 73.406) (width 0.5) (layer "F.Cu") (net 9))
 (segment (start 167.9956 70.3976) (end 173.9204 64.4728) (width 0.5) (layer "F.Cu") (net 5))
 (segment (start 177.6476 52.4764) (end 180.7464 49.3776) (width 0.5) (layer "F.Cu") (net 5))
 (segment (start 173.9204 64.4728) (end 173.9204 54.4764) (width 0.5) (layer "F.Cu") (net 5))
 (segment (start 173.9204 54.4764) (end 175.9204 52.4764) (width 0.5) (layer "F.Cu") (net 5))
 (segment (start 175.9204 52.4764) (end 177.6476 52.4764) (width 0.5) (layer "F.Cu") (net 5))
 (segment (start 178.816 75.220247) (end 178.816 72.5932) (width 0.5) (layer "B.Cu") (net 5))
 (segment (start 199.3392 73.406) (end 199.3392 75.5528) (width 0.5) (layer "B.Cu") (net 5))
 (segment (start 210.5152 73.406) (end 210.5152 75.756) (width 0.5) (layer "B.Cu") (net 5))
 (segment (start 221.9452 73.406) (end 219.5952 75.756) (width 0.5) (layer "B.Cu") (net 5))
 (segment (start 199.5424 75.756) (end 179.351753 75.756) (width 0.5) (layer "B.Cu") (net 5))
 (segment (start 199.3392 75.5528) (end 199.5424 75.756) (width 0.5) (layer "B.Cu") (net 5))
 (segment (start 228.9556 73.406) (end 232.1052 70.2564) (width 0.5) (layer "B.Cu") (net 5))
 (segment (start 210.5152 75.756) (end 199.5424 75.756) (width 0.5) (layer "B.Cu") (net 5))
 (segment (start 179.351753 75.756) (end 178.816 75.220247) (width 0.5) (layer "B.Cu") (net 5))
 (segment (start 178.816 72.5932) (end 176.6204 70.3976) (width 0.5) (layer "B.Cu") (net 5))
 (segment (start 176.6204 70.3976) (end 167.9956 70.3976) (width 0.5) (layer "B.Cu") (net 5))
 (segment (start 219.5952 75.756) (end 210.5152 75.756) (width 0.5) (layer "B.Cu") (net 5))
 (segment (start 221.9452 73.406) (end 228.9556 73.406) (width 0.5) (layer "B.Cu") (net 5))
 (segment (start 158.0488 56.5812) (end 159.4716 55.1584) (width 0.5) (layer "B.Cu") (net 2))
 (segment (start 159.4716 55.1584) (end 159.4716 47.498) (width 0.5) (layer "B.Cu") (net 2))
 (segment (start 158.1912 47.498) (end 158.1912 53.8988) (width 0.5) (layer "F.Cu") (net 3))
 (segment (start 158.1912 53.8988) (end 155.5088 56.5812) (width 0.5) (layer "F.Cu") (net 3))
 (segment (start 147.4724 49.4792) (end 150.876 46.0756) (width 0.5) (layer "F.Cu") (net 18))
 (segment (start 179.364799 45.069601) (end 183.925601 45.069601) (width 0.5) (layer "F.Cu") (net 18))
 (segment (start 178.3588 46.0756) (end 179.364799 45.069601) (width 0.5) (layer "F.Cu") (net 18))
 (segment (start 183.925601 45.069601) (end 184.7256 45.8696) (width 0.5) (layer "F.Cu") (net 18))
 (segment (start 108.971 55.626) (end 108.971 52.790307) (width 0.5) (layer "F.Cu") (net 18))
 (segment (start 112.282107 49.4792) (end 147.4724 49.4792) (width 0.5) (layer "F.Cu") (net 18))
 (segment (start 150.876 46.0756) (end 178.3588 46.0756) (width 0.5) (layer "F.Cu") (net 18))
 (segment (start 108.971 52.790307) (end 112.282107 49.4792) (width 0.5) (layer "F.Cu") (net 18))
 (segment (start 180.715063 61.444627) (end 180.715063 51.880137) (width 0.5) (layer "B.Cu") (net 20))
 (segment (start 180.7464 67.8068) (end 180.7464 61.909908) (width 0.5) (layer "B.Cu") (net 20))
 (segment (start 180.715063 51.880137) (end 186.7256 45.8696) (width 0.5) (layer "B.Cu") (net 20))
 (segment (start 180.7464 61.909908) (end 180.715063 61.444627) (width 0.5) (layer "B.Cu") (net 20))
 (segment (start 180.7464 70.3468) (end 177.1466 73.9466) (width 0.5) (layer "F.Cu") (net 19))
 (segment (start 117.430646 58.518766) (end 117.430646 57.676954) (width 0.5) (layer "F.Cu") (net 19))
 (segment (start 126.746 67.83412) (end 117.430646 58.518766) (width 0.5) (layer "F.Cu") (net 19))
 (segment (start 151.860388 70.2056) (end 126.746 70.2056) (width 0.5) (layer "F.Cu") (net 19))
 (segment (start 126.746 70.2056) (end 126.746 67.83412) (width 0.5) (layer "F.Cu") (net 19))
 (segment (start 155.601388 73.9466) (end 151.860388 70.2056) (width 0.5) (layer "F.Cu") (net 19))
 (segment (start 177.1466 73.9466) (end 155.601388 73.9466) (width 0.5) (layer "F.Cu") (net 19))
 (via (at 117.430646 57.676954) (size 0.6) (drill 0.3) (layers "F.Cu" "B.Cu") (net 19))
 (segment (start 117.430646 51.630661) (end 115.292526 49.492541) (width 0.5) (layer "B.Cu") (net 19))
 (segment (start 106.432547 55.32876) (end 106.432547 55.537355) (width 0.5) (layer "B.Cu") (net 19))
 (segment (start 117.430646 57.676954) (end 117.430646 51.630661) (width 0.5) (layer "B.Cu") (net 19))
 (segment (start 115.292526 49.492541) (end 112.268766 49.492541) (width 0.5) (layer "B.Cu") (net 19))
 (segment (start 112.268766 49.492541) (end 106.432547 55.32876) (width 0.5) (layer "B.Cu") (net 19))
 (segment (start 160.5888 66.6484) (end 164.338 70.3976) (width 0.5) (layer "B.Cu") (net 12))
 (segment (start 160.5888 56.5812) (end 160.5888 66.6484) (width 0.5) (layer "B.Cu") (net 12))
 (segment (start 164.338 57.7904) (end 163.1288 56.5812) (width 0.5) (layer "B.Cu") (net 13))
 (segment (start 164.338 67.8576) (end 164.338 57.7904) (width 0.5) (layer "B.Cu") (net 13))
 (segment (start 163.795922 71.694) (end 163.799522 71.6976) (width 0.5) (layer "F.Cu") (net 4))
 (segment (start 157.3276 72.644) (end 157.3276 72.268) (width 0.5) (layer "F.Cu") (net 4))
 (segment (start 166.2176 70.356478) (end 166.2176 69.6356) (width 0.5) (layer "F.Cu") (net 4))
 (segment (start 157.9016 71.694) (end 163.795922 71.694) (width 0.5) (layer "F.Cu") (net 4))
 (segment (start 157.3276 72.268) (end 157.9016 71.694) (width 0.5) (layer "F.Cu") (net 4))
 (segment (start 163.799522 71.6976) (end 164.876478 71.6976) (width 0.5) (layer "F.Cu") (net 4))
 (segment (start 166.2176 69.6356) (end 167.9956 67.8576) (width 0.5) (layer "F.Cu") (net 4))
 (segment (start 164.876478 71.6976) (end 166.2176 70.356478) (width 0.5) (layer "F.Cu") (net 4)))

